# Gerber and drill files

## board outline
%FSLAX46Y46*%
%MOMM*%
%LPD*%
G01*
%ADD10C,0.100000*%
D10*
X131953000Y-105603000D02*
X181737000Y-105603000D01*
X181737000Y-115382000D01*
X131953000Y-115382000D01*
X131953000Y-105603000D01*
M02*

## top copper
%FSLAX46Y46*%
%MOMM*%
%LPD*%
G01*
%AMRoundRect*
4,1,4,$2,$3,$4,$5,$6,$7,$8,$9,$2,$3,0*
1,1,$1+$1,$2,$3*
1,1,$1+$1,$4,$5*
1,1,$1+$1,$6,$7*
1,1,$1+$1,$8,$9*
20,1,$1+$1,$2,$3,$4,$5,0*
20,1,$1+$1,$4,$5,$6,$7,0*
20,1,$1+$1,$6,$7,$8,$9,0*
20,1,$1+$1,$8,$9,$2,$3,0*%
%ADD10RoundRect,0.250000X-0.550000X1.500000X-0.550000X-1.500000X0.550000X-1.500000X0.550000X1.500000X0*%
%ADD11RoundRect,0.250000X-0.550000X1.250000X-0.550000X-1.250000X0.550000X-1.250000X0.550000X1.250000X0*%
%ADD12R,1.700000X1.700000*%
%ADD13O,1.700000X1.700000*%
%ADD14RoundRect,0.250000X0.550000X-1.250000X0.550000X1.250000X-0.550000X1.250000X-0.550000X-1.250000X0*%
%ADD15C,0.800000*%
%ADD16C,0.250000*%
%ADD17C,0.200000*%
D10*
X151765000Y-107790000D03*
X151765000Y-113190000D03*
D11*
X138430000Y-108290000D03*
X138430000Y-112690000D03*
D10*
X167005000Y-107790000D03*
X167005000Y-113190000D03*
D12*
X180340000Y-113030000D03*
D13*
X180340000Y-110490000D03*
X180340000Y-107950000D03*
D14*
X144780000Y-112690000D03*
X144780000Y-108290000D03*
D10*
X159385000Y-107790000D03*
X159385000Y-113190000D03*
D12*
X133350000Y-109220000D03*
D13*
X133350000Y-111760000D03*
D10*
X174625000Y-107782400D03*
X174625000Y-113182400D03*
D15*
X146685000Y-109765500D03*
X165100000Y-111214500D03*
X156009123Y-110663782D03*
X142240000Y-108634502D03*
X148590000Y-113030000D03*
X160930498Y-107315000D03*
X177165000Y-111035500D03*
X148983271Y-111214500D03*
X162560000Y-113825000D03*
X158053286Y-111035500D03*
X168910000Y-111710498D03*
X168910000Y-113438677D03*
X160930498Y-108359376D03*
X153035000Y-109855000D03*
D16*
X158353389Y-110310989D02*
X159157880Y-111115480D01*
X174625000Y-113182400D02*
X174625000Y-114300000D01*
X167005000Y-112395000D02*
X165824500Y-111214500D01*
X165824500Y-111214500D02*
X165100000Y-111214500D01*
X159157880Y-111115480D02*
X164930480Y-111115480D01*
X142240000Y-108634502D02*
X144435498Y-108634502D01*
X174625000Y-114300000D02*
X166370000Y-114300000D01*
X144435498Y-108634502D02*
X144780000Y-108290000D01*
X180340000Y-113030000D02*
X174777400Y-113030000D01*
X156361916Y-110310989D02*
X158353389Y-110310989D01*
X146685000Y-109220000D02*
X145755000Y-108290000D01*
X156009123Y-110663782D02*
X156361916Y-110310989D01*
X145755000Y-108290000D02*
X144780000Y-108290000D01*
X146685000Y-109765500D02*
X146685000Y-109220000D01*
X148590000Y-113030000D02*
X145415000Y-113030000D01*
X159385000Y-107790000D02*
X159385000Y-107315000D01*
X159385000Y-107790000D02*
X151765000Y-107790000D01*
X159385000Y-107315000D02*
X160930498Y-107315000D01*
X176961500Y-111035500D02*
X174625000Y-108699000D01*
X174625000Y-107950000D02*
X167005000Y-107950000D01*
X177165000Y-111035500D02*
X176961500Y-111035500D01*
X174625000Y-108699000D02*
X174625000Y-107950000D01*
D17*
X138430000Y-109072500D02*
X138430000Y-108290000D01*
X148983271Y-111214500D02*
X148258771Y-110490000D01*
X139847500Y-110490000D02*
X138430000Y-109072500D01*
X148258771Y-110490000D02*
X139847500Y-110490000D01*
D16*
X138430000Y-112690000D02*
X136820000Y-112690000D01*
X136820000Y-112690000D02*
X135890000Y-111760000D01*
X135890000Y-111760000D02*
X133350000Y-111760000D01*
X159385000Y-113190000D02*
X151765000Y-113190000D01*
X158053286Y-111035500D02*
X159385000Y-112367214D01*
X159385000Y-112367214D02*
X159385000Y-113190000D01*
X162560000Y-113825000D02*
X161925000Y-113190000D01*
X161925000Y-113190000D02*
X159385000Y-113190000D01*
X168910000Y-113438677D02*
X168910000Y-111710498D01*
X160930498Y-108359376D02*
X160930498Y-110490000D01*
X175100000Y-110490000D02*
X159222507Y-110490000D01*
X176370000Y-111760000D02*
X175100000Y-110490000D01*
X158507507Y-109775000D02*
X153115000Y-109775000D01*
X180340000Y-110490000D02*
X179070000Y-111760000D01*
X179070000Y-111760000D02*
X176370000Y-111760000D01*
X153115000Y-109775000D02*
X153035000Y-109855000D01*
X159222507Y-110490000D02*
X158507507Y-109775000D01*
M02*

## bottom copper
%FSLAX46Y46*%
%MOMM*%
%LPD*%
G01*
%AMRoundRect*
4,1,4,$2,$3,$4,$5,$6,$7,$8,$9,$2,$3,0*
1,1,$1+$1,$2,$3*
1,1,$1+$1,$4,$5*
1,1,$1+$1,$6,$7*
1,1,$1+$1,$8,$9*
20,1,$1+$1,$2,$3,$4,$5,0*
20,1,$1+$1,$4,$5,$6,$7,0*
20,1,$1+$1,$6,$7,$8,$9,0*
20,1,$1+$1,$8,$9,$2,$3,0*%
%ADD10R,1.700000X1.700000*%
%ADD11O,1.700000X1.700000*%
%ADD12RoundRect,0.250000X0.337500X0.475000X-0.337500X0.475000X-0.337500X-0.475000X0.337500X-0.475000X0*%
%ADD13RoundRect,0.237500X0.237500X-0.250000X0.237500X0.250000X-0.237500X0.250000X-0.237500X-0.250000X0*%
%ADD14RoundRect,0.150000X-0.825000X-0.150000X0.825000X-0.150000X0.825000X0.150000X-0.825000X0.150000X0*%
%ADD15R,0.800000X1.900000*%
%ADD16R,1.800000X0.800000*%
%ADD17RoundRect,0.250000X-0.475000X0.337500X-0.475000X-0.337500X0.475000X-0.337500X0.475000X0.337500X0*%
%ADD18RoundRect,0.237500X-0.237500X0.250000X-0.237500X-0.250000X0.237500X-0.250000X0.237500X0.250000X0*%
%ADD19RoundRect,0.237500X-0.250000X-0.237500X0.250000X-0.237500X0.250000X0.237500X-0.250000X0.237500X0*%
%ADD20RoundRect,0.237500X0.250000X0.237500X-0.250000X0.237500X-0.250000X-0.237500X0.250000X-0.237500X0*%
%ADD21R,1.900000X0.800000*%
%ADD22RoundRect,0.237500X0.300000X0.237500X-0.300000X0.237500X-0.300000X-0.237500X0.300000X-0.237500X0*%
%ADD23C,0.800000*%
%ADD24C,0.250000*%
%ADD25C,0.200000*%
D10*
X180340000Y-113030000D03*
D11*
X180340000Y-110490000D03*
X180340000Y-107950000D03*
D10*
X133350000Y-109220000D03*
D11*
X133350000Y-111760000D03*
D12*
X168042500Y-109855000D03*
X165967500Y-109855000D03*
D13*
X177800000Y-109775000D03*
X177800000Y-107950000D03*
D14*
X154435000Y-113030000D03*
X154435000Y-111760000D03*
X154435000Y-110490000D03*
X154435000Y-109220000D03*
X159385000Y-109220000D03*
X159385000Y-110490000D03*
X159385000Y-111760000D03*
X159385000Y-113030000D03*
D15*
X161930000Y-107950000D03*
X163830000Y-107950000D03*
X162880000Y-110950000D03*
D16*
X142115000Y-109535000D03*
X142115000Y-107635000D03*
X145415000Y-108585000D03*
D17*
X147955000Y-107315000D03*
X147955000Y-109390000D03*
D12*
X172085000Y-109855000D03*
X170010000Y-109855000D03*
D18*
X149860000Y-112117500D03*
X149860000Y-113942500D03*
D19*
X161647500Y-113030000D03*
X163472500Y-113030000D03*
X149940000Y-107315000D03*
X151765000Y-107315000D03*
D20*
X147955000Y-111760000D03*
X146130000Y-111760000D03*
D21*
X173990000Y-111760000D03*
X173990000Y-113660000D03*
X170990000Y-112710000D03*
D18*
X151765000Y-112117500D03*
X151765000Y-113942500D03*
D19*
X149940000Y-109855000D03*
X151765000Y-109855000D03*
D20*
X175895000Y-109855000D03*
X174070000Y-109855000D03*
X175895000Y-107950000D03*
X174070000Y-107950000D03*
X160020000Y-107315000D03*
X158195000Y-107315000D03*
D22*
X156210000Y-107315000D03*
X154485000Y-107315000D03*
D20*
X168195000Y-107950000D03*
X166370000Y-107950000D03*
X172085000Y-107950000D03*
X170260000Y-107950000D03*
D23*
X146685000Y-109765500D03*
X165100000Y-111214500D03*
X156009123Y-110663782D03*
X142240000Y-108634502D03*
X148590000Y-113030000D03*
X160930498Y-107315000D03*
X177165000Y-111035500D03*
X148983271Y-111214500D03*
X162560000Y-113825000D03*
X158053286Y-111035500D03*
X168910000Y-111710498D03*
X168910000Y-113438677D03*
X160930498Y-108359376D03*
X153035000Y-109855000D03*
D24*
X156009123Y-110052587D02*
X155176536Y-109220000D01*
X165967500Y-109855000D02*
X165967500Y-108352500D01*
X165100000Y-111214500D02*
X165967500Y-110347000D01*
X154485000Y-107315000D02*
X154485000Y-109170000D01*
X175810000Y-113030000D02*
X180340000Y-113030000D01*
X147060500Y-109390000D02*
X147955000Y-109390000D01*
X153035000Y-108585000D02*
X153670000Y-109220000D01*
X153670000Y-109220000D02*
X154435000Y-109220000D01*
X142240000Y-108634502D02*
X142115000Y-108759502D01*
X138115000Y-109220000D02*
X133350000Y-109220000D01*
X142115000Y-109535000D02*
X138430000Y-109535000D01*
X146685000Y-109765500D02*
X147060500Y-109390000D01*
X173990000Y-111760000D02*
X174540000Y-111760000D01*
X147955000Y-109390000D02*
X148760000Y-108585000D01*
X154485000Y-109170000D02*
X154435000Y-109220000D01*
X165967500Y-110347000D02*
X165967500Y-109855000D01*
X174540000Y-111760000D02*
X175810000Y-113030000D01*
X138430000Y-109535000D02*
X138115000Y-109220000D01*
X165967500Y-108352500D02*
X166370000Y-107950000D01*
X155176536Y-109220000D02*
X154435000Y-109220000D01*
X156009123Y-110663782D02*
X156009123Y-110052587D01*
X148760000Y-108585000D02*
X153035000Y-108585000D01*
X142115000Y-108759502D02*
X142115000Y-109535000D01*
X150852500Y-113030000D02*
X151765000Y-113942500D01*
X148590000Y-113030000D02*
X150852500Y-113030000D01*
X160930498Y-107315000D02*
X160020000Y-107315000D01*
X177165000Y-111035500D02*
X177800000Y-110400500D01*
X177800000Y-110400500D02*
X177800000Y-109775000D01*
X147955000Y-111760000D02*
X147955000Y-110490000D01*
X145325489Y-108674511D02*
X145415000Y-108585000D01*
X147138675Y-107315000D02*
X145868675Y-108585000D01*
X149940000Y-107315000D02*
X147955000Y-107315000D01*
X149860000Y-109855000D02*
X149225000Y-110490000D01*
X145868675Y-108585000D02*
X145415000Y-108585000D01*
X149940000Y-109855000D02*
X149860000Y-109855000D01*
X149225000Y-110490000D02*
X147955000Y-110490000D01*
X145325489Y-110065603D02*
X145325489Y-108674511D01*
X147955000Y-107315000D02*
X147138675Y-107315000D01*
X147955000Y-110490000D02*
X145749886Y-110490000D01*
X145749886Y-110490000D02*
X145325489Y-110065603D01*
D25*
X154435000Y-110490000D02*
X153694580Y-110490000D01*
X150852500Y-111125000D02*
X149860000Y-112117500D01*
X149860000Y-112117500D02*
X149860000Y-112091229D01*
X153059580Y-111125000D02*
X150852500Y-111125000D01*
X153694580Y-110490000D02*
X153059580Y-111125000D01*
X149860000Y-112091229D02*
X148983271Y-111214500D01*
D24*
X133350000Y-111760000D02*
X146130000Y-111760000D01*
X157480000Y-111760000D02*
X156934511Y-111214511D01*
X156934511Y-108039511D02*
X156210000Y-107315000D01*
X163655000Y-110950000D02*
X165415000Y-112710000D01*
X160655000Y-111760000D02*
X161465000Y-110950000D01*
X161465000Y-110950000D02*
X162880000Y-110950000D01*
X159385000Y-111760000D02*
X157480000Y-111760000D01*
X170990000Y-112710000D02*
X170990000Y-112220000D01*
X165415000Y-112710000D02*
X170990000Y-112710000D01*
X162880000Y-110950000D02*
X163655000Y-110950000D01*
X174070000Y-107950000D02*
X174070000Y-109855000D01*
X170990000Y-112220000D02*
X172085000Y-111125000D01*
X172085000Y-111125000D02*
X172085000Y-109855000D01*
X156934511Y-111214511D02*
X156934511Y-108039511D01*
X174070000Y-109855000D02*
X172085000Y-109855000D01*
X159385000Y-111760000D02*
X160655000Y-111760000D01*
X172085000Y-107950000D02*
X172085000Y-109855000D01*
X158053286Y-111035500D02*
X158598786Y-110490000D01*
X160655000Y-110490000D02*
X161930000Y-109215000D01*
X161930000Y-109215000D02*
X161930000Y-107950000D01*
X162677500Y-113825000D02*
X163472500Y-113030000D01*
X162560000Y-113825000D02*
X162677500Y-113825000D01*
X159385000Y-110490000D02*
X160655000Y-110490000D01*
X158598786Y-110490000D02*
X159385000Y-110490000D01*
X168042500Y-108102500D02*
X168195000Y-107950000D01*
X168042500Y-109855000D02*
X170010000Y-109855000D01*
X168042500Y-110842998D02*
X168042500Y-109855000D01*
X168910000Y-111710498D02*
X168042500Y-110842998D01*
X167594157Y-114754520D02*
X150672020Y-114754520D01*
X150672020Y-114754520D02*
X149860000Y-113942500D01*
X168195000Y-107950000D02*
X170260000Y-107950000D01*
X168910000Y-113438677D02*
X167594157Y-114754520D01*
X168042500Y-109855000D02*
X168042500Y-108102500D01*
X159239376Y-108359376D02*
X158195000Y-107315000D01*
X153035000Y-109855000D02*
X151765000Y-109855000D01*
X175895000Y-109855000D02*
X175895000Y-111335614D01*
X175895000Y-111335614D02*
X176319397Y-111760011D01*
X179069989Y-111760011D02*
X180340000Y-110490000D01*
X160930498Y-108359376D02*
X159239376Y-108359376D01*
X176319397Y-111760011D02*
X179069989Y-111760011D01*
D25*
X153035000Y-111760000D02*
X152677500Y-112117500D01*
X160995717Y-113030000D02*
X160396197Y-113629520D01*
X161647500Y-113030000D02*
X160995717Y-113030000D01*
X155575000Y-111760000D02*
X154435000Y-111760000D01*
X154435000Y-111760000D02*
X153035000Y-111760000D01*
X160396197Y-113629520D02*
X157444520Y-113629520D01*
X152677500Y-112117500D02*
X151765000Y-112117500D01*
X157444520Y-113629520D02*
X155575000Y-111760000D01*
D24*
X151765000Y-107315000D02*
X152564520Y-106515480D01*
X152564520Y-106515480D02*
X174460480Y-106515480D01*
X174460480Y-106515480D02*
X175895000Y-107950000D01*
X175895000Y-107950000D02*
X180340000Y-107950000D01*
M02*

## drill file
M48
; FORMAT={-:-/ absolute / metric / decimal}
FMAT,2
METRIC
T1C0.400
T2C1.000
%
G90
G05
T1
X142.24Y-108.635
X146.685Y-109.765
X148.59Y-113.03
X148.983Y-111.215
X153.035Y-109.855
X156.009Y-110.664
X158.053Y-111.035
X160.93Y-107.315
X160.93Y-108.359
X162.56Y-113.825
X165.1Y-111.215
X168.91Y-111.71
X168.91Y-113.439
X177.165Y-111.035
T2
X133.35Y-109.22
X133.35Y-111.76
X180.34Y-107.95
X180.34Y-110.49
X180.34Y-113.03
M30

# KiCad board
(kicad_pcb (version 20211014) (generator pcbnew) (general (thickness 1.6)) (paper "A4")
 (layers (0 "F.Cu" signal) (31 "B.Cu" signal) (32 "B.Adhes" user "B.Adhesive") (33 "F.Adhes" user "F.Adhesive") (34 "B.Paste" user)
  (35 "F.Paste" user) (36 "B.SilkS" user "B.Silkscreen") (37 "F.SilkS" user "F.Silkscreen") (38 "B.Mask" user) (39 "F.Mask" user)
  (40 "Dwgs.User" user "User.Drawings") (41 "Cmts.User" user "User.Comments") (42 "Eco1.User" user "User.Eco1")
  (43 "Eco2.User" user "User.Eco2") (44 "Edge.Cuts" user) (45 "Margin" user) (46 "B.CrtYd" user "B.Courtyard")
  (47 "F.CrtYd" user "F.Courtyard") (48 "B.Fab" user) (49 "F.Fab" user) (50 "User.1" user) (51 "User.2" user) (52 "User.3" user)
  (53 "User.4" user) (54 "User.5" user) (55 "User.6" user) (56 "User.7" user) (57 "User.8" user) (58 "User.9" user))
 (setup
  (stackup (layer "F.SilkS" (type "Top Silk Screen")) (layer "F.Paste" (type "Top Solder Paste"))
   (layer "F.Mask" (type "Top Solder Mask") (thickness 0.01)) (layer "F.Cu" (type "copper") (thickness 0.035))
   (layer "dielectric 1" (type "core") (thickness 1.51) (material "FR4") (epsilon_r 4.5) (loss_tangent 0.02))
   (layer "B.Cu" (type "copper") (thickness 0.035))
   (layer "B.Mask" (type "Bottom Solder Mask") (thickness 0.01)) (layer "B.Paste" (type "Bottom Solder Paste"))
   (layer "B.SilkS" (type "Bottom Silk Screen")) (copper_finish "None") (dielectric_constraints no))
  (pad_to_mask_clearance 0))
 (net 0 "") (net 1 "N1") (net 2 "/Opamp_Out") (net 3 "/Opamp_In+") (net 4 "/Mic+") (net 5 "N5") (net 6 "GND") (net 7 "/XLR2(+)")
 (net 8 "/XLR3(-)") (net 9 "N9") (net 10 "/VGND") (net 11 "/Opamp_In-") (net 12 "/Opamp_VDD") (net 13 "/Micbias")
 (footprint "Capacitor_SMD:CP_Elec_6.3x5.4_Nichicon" (layer "F.Cu") (at 151.765 110.49 -90)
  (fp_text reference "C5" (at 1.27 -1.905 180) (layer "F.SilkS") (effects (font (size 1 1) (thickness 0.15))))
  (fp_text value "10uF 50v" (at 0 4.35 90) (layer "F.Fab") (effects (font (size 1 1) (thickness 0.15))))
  (pad "1" smd roundrect (at -2.7 0 270) (size 3.5 1.6) (layers "F.Cu" "F.Paste" "F.Mask") (roundrect_rratio 0.15625) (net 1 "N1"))
  (pad "2" smd roundrect (at 2.7 0 270) (size 3.5 1.6) (layers "F.Cu" "F.Paste" "F.Mask") (roundrect_rratio 0.15625) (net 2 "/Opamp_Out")))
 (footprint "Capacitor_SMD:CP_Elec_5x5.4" (layer "F.Cu") (at 138.43 110.49 -90)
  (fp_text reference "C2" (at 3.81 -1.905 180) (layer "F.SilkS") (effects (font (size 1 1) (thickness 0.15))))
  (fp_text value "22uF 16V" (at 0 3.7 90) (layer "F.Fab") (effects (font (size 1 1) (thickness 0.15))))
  (pad "1" smd roundrect (at -2.2 0 270) (size 3 1.6) (layers "F.Cu" "F.Paste" "F.Mask") (roundrect_rratio 0.15625) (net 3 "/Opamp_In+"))
  (pad "2" smd roundrect (at 2.2 0 270) (size 3 1.6) (layers "F.Cu" "F.Paste" "F.Mask") (roundrect_rratio 0.15625) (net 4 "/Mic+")))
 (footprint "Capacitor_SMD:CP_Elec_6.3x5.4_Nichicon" (layer "F.Cu") (at 167.005 110.49 -90)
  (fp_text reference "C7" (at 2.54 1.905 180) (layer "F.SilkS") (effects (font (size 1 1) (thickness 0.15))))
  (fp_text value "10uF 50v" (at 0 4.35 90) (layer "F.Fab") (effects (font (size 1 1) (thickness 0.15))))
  (pad "1" smd roundrect (at -2.7 0 270) (size 3.5 1.6) (layers "F.Cu" "F.Paste" "F.Mask") (roundrect_rratio 0.15625) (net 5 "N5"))
  (pad "2" smd roundrect (at 2.7 0 270) (size 3.5 1.6) (layers "F.Cu" "F.Paste" "F.Mask") (roundrect_rratio 0.15625) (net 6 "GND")))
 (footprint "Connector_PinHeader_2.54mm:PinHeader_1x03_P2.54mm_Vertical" (layer "F.Cu") (at 180.34 113.03 180)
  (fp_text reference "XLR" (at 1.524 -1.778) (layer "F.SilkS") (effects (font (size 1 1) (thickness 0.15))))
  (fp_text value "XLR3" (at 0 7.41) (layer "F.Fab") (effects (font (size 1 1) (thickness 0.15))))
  (pad "1" thru_hole rect (at 0 0 180) (size 1.7 1.7) (drill 1) (layers *.Cu *.Mask) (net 6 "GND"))
  (pad "2" thru_hole oval (at 0 2.54 180) (size 1.7 1.7) (drill 1) (layers *.Cu *.Mask) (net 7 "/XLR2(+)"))
  (pad "3" thru_hole oval (at 0 5.08 180) (size 1.7 1.7) (drill 1) (layers *.Cu *.Mask) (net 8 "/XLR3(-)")))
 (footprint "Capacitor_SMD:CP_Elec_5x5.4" (layer "F.Cu") (at 144.78 110.49 90)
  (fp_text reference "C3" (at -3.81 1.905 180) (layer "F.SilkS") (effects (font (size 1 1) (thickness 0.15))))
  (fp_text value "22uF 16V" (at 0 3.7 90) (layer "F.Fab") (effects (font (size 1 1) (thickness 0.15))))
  (pad "1" smd roundrect (at -2.2 0 90) (size 3 1.6) (layers "F.Cu" "F.Paste" "F.Mask") (roundrect_rratio 0.15625) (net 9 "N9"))
  (pad "2" smd roundrect (at 2.2 0 90) (size 3 1.6) (layers "F.Cu" "F.Paste" "F.Mask") (roundrect_rratio 0.15625) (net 6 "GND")))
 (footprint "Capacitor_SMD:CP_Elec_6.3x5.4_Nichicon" (layer "F.Cu") (at 159.385 110.49 -90)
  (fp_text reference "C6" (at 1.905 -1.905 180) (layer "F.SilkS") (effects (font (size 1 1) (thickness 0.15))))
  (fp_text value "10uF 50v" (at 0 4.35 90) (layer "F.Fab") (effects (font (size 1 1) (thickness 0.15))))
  (pad "1" smd roundrect (at -2.7 0 270) (size 3.5 1.6) (layers "F.Cu" "F.Paste" "F.Mask") (roundrect_rratio 0.15625) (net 1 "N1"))
  (pad "2" smd roundrect (at 2.7 0 270) (size 3.5 1.6) (layers "F.Cu" "F.Paste" "F.Mask") (roundrect_rratio 0.15625) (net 2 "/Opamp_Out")))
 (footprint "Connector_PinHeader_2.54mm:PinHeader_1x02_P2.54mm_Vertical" (layer "F.Cu") (at 133.35 109.22)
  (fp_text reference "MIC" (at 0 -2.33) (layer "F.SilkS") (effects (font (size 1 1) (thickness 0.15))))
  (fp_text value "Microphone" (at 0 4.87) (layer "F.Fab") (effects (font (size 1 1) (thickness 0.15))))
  (pad "1" thru_hole rect (at 0 0) (size 1.7 1.7) (drill 1) (layers *.Cu *.Mask) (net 6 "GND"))
  (pad "2" thru_hole oval (at 0 2.54) (size 1.7 1.7) (drill 1) (layers *.Cu *.Mask) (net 4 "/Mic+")))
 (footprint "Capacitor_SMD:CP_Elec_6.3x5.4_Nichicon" (layer "F.Cu") (at 174.625 110.4824 -90)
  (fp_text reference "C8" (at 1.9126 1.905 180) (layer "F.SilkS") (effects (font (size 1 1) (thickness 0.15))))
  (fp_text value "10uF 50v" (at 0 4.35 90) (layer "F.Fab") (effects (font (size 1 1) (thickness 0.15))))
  (pad "1" smd roundrect (at -2.7 0 270) (size 3.5 1.6) (layers "F.Cu" "F.Paste" "F.Mask") (roundrect_rratio 0.15625) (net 5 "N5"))
  (pad "2" smd roundrect (at 2.7 0 270) (size 3.5 1.6) (layers "F.Cu" "F.Paste" "F.Mask") (roundrect_rratio 0.15625) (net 6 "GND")))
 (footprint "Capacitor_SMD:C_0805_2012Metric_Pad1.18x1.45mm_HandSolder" (layer "B.Cu") (at 167.005 109.855 180)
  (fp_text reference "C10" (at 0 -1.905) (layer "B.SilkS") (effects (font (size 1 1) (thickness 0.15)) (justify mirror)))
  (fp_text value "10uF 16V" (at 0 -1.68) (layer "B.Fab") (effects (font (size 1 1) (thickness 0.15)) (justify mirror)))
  (pad "1" smd roundrect (at -1.0375 0 180) (size 1.175 1.45) (layers "B.Cu" "B.Paste" "B.Mask") (roundrect_rratio 0.2127659574)
   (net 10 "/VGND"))
  (pad "2" smd roundrect (at 1.0375 0 180) (size 1.175 1.45) (layers "B.Cu" "B.Paste" "B.Mask") (roundrect_rratio 0.2127659574)
   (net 6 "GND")))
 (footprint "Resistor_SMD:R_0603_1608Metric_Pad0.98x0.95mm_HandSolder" (layer "B.Cu") (at 177.8 108.8625 90)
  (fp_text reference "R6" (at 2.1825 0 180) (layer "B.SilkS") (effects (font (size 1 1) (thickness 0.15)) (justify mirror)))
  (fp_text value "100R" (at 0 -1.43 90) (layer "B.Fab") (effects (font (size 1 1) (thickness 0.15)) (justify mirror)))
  (pad "1" smd roundrect (at -0.9125 0 90) (size 0.975 0.95) (layers "B.Cu" "B.Paste" "B.Mask") (roundrect_rratio 0.25) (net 5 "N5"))
  (pad "2" smd roundrect (at 0.9125 0 90) (size 0.975 0.95) (layers "B.Cu" "B.Paste" "B.Mask") (roundrect_rratio 0.25) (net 8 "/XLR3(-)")))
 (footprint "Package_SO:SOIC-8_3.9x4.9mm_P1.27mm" (layer "B.Cu") (at 156.91 111.125)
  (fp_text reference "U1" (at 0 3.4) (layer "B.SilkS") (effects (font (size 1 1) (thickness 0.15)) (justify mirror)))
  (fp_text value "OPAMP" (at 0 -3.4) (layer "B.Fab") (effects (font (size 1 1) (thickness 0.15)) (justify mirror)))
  (pad "1" smd roundrect (at -2.475 1.905) (size 1.95 0.6) (layers "B.Cu" "B.Paste" "B.Mask") (roundrect_rratio 0.25))
  (pad "2" smd roundrect (at -2.475 0.635) (size 1.95 0.6) (layers "B.Cu" "B.Paste" "B.Mask") (roundrect_rratio 0.25) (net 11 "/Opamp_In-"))
  (pad "3" smd roundrect (at -2.475 -0.635) (size 1.95 0.6) (layers "B.Cu" "B.Paste" "B.Mask") (roundrect_rratio 0.25) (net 3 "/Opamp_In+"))
  (pad "4" smd roundrect (at -2.475 -1.905) (size 1.95 0.6) (layers "B.Cu" "B.Paste" "B.Mask") (roundrect_rratio 0.25) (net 6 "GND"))
  (pad "5" smd roundrect (at 2.475 -1.905) (size 1.95 0.6) (layers "B.Cu" "B.Paste" "B.Mask") (roundrect_rratio 0.25))
  (pad "6" smd roundrect (at 2.475 -0.635) (size 1.95 0.6) (layers "B.Cu" "B.Paste" "B.Mask") (roundrect_rratio 0.25) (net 2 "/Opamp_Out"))
  (pad "7" smd roundrect (at 2.475 0.635) (size 1.95 0.6) (layers "B.Cu" "B.Paste" "B.Mask") (roundrect_rratio 0.25) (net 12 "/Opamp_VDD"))
  (pad "8" smd roundrect (at 2.475 1.905) (size 1.95 0.6) (layers "B.Cu" "B.Paste" "B.Mask") (roundrect_rratio 0.25)))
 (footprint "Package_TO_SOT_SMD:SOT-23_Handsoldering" (layer "B.Cu") (at 162.88 109.45 -90)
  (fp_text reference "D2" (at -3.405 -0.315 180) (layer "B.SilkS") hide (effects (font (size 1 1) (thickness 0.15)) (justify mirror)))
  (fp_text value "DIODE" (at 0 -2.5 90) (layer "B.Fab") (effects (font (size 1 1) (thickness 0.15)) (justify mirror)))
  (pad "1" smd rect (at -1.5 0.95 270) (size 1.9 0.8) (layers "B.Cu" "B.Paste" "B.Mask") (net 2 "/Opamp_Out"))
  (pad "2" smd rect (at -1.5 -0.95 270) (size 1.9 0.8) (layers "B.Cu" "B.Paste" "B.Mask"))
  (pad "3" smd rect (at 1.5 0 270) (size 1.9 0.8) (layers "B.Cu" "B.Paste" "B.Mask") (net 12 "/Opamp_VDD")))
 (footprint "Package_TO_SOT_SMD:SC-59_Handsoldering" (layer "B.Cu") (at 143.765 108.585)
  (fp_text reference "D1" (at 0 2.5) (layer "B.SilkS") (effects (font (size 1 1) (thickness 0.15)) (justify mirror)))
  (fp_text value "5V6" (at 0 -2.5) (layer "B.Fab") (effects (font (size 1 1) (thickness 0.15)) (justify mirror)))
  (pad "1" smd rect (at -1.65 0.95) (size 1.8 0.8) (layers "B.Cu" "B.Paste" "B.Mask") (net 6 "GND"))
  (pad "2" smd rect (at -1.65 -0.95) (size 1.8 0.8) (layers "B.Cu" "B.Paste" "B.Mask"))
  (pad "3" smd rect (at 1.65 0) (size 1.8 0.8) (layers "B.Cu" "B.Paste" "B.Mask") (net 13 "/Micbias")))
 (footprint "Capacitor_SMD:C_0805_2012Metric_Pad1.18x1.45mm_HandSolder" (layer "B.Cu") (at 147.955 108.3525 -90)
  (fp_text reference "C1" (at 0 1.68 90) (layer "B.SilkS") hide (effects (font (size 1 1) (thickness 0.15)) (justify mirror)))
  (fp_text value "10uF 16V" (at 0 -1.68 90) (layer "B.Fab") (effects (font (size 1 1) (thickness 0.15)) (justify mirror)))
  (pad "1" smd roundrect (at -1.0375 0 270) (size 1.175 1.45) (layers "B.Cu" "B.Paste" "B.Mask") (roundrect_rratio 0.2127659574)
   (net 13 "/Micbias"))
  (pad "2" smd roundrect (at 1.0375 0 270) (size 1.175 1.45) (layers "B.Cu" "B.Paste" "B.Mask") (roundrect_rratio 0.2127659574)
   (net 6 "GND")))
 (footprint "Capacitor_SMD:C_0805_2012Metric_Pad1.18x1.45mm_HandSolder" (layer "B.Cu") (at 171.0475 109.855 180)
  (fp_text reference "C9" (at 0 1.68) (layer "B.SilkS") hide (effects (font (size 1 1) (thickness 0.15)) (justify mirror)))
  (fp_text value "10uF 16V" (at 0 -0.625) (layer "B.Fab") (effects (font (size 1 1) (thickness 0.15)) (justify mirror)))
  (pad "1" smd roundrect (at -1.0375 0 180) (size 1.175 1.45) (layers "B.Cu" "B.Paste" "B.Mask") (roundrect_rratio 0.2127659574)
   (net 12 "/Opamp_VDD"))
  (pad "2" smd roundrect (at 1.0375 0 180) (size 1.175 1.45) (layers "B.Cu" "B.Paste" "B.Mask") (roundrect_rratio 0.2127659574)
   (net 10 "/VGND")))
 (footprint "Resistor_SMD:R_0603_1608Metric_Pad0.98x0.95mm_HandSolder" (layer "B.Cu") (at 149.86 113.03 -90)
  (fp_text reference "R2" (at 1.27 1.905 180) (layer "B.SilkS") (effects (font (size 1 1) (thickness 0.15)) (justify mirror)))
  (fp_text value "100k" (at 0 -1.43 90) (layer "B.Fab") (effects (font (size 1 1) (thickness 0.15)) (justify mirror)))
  (pad "1" smd roundrect (at -0.9125 0 270) (size 0.975 0.95) (layers "B.Cu" "B.Paste" "B.Mask") (roundrect_rratio 0.25)
   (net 3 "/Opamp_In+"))
  (pad "2" smd roundrect (at 0.9125 0 270) (size 0.975 0.95) (layers "B.Cu" "B.Paste" "B.Mask") (roundrect_rratio 0.25) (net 10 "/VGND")))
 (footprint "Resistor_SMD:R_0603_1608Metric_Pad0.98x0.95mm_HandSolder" (layer "B.Cu") (at 162.56 113.03)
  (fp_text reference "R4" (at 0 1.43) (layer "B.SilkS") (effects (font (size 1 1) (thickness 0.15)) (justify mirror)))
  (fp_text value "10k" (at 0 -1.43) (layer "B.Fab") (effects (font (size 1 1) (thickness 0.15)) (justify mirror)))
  (pad "1" smd roundrect (at -0.9125 0) (size 0.975 0.95) (layers "B.Cu" "B.Paste" "B.Mask") (roundrect_rratio 0.25) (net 11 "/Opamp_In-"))
  (pad "2" smd roundrect (at 0.9125 0) (size 0.975 0.95) (layers "B.Cu" "B.Paste" "B.Mask") (roundrect_rratio 0.25) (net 2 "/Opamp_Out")))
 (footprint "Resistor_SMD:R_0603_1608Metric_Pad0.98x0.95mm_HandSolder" (layer "B.Cu") (at 150.8525 107.315)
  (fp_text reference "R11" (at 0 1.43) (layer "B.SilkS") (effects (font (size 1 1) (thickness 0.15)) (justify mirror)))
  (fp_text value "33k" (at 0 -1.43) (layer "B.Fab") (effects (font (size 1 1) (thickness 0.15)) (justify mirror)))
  (pad "1" smd roundrect (at -0.9125 0) (size 0.975 0.95) (layers "B.Cu" "B.Paste" "B.Mask") (roundrect_rratio 0.25) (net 13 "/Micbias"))
  (pad "2" smd roundrect (at 0.9125 0) (size 0.975 0.95) (layers "B.Cu" "B.Paste" "B.Mask") (roundrect_rratio 0.25) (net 8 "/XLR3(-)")))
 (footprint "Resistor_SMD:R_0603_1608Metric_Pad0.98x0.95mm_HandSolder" (layer "B.Cu") (at 147.0425 111.76 180)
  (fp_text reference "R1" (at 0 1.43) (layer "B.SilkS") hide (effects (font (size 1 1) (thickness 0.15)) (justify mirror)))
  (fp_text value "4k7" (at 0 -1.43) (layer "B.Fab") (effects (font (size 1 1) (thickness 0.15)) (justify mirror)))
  (pad "1" smd roundrect (at -0.9125 0 180) (size 0.975 0.95) (layers "B.Cu" "B.Paste" "B.Mask") (roundrect_rratio 0.25) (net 13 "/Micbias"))
  (pad "2" smd roundrect (at 0.9125 0 180) (size 0.975 0.95) (layers "B.Cu" "B.Paste" "B.Mask") (roundrect_rratio 0.25) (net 4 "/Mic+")))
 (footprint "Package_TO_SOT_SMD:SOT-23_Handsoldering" (layer "B.Cu") (at 172.49 112.71 180)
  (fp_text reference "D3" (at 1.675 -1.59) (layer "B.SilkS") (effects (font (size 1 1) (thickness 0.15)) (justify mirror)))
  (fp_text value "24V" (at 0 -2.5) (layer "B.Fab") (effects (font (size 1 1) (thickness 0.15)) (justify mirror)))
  (pad "1" smd rect (at -1.5 0.95 180) (size 1.9 0.8) (layers "B.Cu" "B.Paste" "B.Mask") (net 6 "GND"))
  (pad "2" smd rect (at -1.5 -0.95 180) (size 1.9 0.8) (layers "B.Cu" "B.Paste" "B.Mask"))
  (pad "3" smd rect (at 1.5 0 180) (size 1.9 0.8) (layers "B.Cu" "B.Paste" "B.Mask") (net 12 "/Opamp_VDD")))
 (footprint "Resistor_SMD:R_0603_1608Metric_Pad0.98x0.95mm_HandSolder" (layer "B.Cu") (at 151.765 113.03 -90)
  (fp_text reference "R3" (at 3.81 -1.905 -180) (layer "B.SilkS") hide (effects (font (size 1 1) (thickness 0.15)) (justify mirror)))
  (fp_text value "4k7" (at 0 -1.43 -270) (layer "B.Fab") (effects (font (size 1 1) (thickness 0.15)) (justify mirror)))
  (pad "1" smd roundrect (at -0.9125 0 270) (size 0.975 0.95) (layers "B.Cu" "B.Paste" "B.Mask") (roundrect_rratio 0.25)
   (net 11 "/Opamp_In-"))
  (pad "2" smd roundrect (at 0.9125 0 270) (size 0.975 0.95) (layers "B.Cu" "B.Paste" "B.Mask") (roundrect_rratio 0.25) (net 9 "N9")))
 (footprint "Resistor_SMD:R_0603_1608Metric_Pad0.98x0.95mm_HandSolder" (layer "B.Cu") (at 150.8525 109.855)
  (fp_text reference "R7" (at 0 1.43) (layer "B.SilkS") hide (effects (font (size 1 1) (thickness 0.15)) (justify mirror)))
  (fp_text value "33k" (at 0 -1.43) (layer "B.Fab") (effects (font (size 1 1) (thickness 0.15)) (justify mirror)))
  (pad "1" smd roundrect (at -0.9125 0) (size 0.975 0.95) (layers "B.Cu" "B.Paste" "B.Mask") (roundrect_rratio 0.25) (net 13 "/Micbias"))
  (pad "2" smd roundrect (at 0.9125 0) (size 0.975 0.95) (layers "B.Cu" "B.Paste" "B.Mask") (roundrect_rratio 0.25) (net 7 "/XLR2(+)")))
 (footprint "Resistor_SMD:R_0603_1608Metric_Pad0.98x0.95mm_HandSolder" (layer "B.Cu") (at 174.9825 109.855 180)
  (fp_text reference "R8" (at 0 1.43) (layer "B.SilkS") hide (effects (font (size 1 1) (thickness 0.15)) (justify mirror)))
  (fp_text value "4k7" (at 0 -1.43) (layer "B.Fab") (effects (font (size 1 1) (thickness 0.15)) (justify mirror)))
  (pad "1" smd roundrect (at -0.9125 0 180) (size 0.975 0.95) (layers "B.Cu" "B.Paste" "B.Mask") (roundrect_rratio 0.25) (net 7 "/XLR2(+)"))
  (pad "2" smd roundrect (at 0.9125 0 180) (size 0.975 0.95) (layers "B.Cu" "B.Paste" "B.Mask") (roundrect_rratio 0.25)
   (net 12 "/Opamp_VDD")))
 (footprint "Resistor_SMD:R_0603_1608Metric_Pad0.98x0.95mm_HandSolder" (layer "B.Cu") (at 174.9825 107.95 180)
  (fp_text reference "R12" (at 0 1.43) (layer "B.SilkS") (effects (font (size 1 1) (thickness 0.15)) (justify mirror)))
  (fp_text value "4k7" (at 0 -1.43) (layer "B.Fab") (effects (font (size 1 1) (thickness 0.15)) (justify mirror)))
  (pad "1" smd roundrect (at -0.9125 0 180) (size 0.975 0.95) (layers "B.Cu" "B.Paste" "B.Mask") (roundrect_rratio 0.25) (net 8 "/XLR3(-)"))
  (pad "2" smd roundrect (at 0.9125 0 180) (size 0.975 0.95) (layers "B.Cu" "B.Paste" "B.Mask") (roundrect_rratio 0.25)
   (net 12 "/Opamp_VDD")))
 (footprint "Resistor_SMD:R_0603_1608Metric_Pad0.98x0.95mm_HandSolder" (layer "B.Cu") (at 159.1075 107.315 180)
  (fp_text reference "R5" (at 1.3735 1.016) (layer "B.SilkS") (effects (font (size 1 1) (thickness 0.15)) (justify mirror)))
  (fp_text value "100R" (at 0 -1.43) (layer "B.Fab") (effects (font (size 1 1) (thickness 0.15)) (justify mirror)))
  (pad "1" smd roundrect (at -0.9125 0 180) (size 0.975 0.95) (layers "B.Cu" "B.Paste" "B.Mask") (roundrect_rratio 0.25) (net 1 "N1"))
  (pad "2" smd roundrect (at 0.9125 0 180) (size 0.975 0.95) (layers "B.Cu" "B.Paste" "B.Mask") (roundrect_rratio 0.25) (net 7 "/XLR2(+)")))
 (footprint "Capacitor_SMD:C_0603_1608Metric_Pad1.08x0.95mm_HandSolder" (layer "B.Cu") (at 155.3475 107.315 180)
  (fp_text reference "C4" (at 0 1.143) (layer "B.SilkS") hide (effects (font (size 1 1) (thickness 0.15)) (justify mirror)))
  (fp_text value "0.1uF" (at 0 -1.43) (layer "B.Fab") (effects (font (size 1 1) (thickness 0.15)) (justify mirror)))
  (pad "1" smd roundrect (at -0.8625 0 180) (size 1.075 0.95) (layers "B.Cu" "B.Paste" "B.Mask") (roundrect_rratio 0.25)
   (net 12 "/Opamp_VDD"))
  (pad "2" smd roundrect (at 0.8625 0 180) (size 1.075 0.95) (layers "B.Cu" "B.Paste" "B.Mask") (roundrect_rratio 0.25) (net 6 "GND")))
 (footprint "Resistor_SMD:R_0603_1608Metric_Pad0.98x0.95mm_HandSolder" (layer "B.Cu") (at 167.2825 107.95 180)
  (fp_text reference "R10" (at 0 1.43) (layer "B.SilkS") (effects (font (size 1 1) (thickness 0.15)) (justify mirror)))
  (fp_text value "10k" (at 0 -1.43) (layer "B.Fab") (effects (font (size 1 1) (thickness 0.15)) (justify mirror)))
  (pad "1" smd roundrect (at -0.9125 0 180) (size 0.975 0.95) (layers "B.Cu" "B.Paste" "B.Mask") (roundrect_rratio 0.25) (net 10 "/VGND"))
  (pad "2" smd roundrect (at 0.9125 0 180) (size 0.975 0.95) (layers "B.Cu" "B.Paste" "B.Mask") (roundrect_rratio 0.25) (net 6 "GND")))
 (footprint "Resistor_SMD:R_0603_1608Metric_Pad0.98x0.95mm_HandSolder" (layer "B.Cu") (at 171.1725 107.95 180)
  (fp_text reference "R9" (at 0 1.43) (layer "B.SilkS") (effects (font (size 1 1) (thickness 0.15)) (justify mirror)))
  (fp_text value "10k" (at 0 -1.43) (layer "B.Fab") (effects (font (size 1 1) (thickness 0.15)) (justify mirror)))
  (pad "1" smd roundrect (at -0.9125 0 180) (size 0.975 0.95) (layers "B.Cu" "B.Paste" "B.Mask") (roundrect_rratio 0.25)
   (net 12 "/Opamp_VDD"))
  (pad "2" smd roundrect (at 0.9125 0 180) (size 0.975 0.95) (layers "B.Cu" "B.Paste" "B.Mask") (roundrect_rratio 0.25) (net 10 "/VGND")))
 (gr_rect (start 131.953 105.603) (end 181.737 115.382) (layer "Edge.Cuts") (width 0.1) (fill none))
 (segment (start 158.353389 110.310989) (end 159.15788 111.11548) (width 0.25) (layer "F.Cu") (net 6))
 (segment (start 174.625 113.1824) (end 174.625 114.3) (width 0.25) (layer "F.Cu") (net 6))
 (segment (start 167.005 112.395) (end 165.8245 111.2145) (width 0.25) (layer "F.Cu") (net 6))
 (segment (start 165.8245 111.2145) (end 165.1 111.2145) (width 0.25) (layer "F.Cu") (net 6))
 (segment (start 159.15788 111.11548) (end 164.93048 111.11548) (width 0.25) (layer "F.Cu") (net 6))
 (segment (start 142.24 108.634502) (end 144.435498 108.634502) (width 0.25) (layer "F.Cu") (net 6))
 (segment (start 174.625 114.3) (end 166.37 114.3) (width 0.25) (layer "F.Cu") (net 6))
 (segment (start 144.435498 108.634502) (end 144.78 108.29) (width 0.25) (layer "F.Cu") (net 6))
 (segment (start 180.34 113.03) (end 174.7774 113.03) (width 0.25) (layer "F.Cu") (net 6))
 (segment (start 156.361916 110.310989) (end 158.353389 110.310989) (width 0.25) (layer "F.Cu") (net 6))
 (segment (start 146.685 109.22) (end 145.755 108.29) (width 0.25) (layer "F.Cu") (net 6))
 (segment (start 156.009123 110.663782) (end 156.361916 110.310989) (width 0.25) (layer "F.Cu") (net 6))
 (segment (start 145.755 108.29) (end 144.78 108.29) (width 0.25) (layer "F.Cu") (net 6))
 (segment (start 146.685 109.7655) (end 146.685 109.22) (width 0.25) (layer "F.Cu") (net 6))
 (via (at 146.685 109.7655) (size 0.8) (drill 0.4) (layers "F.Cu" "B.Cu") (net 6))
 (via (at 165.1 111.2145) (size 0.8) (drill 0.4) (layers "F.Cu" "B.Cu") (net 6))
 (via (at 156.009123 110.663782) (size 0.8) (drill 0.4) (layers "F.Cu" "B.Cu") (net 6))
 (via (at 142.24 108.634502) (size 0.8) (drill 0.4) (layers "F.Cu" "B.Cu") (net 6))
 (segment (start 156.009123 110.052587) (end 155.176536 109.22) (width 0.25) (layer "B.Cu") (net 6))
 (segment (start 165.9675 109.855) (end 165.9675 108.3525) (width 0.25) (layer "B.Cu") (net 6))
 (segment (start 165.1 111.2145) (end 165.9675 110.347) (width 0.25) (layer "B.Cu") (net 6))
 (segment (start 154.485 107.315) (end 154.485 109.17) (width 0.25) (layer "B.Cu") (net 6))
 (segment (start 175.81 113.03) (end 180.34 113.03) (width 0.25) (layer "B.Cu") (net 6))
 (segment (start 147.0605 109.39) (end 147.955 109.39) (width 0.25) (layer "B.Cu") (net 6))
 (segment (start 153.035 108.585) (end 153.67 109.22) (width 0.25) (layer "B.Cu") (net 6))
 (segment (start 153.67 109.22) (end 154.435 109.22) (width 0.25) (layer "B.Cu") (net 6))
 (segment (start 142.24 108.634502) (end 142.115 108.759502) (width 0.25) (layer "B.Cu") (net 6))
 (segment (start 138.115 109.22) (end 133.35 109.22) (width 0.25) (layer "B.Cu") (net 6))
 (segment (start 142.115 109.535) (end 138.43 109.535) (width 0.25) (layer "B.Cu") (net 6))
 (segment (start 146.685 109.7655) (end 147.0605 109.39) (width 0.25) (layer "B.Cu") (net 6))
 (segment (start 173.99 111.76) (end 174.54 111.76) (width 0.25) (layer "B.Cu") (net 6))
 (segment (start 147.955 109.39) (end 148.76 108.585) (width 0.25) (layer "B.Cu") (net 6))
 (segment (start 154.485 109.17) (end 154.435 109.22) (width 0.25) (layer "B.Cu") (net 6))
 (segment (start 165.9675 110.347) (end 165.9675 109.855) (width 0.25) (layer "B.Cu") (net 6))
 (segment (start 174.54 111.76) (end 175.81 113.03) (width 0.25) (layer "B.Cu") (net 6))
 (segment (start 138.43 109.535) (end 138.115 109.22) (width 0.25) (layer "B.Cu") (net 6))
 (segment (start 165.9675 108.3525) (end 166.37 107.95) (width 0.25) (layer "B.Cu") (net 6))
 (segment (start 155.176536 109.22) (end 154.435 109.22) (width 0.25) (layer "B.Cu") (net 6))
 (segment (start 156.009123 110.663782) (end 156.009123 110.052587) (width 0.25) (layer "B.Cu") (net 6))
 (segment (start 148.76 108.585) (end 153.035 108.585) (width 0.25) (layer "B.Cu") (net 6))
 (segment (start 142.115 108.759502) (end 142.115 109.535) (width 0.25) (layer "B.Cu") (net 6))
 (segment (start 148.59 113.03) (end 145.415 113.03) (width 0.25) (layer "F.Cu") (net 9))
 (via (at 148.59 113.03) (size 0.8) (drill 0.4) (layers "F.Cu" "B.Cu") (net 9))
 (segment (start 150.8525 113.03) (end 151.765 113.9425) (width 0.25) (layer "B.Cu") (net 9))
 (segment (start 148.59 113.03) (end 150.8525 113.03) (width 0.25) (layer "B.Cu") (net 9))
 (segment (start 159.385 107.79) (end 159.385 107.315) (width 0.25) (layer "F.Cu") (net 1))
 (segment (start 159.385 107.79) (end 151.765 107.79) (width 0.25) (layer "F.Cu") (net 1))
 (segment (start 159.385 107.315) (end 160.930498 107.315) (width 0.25) (layer "F.Cu") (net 1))
 (via (at 160.930498 107.315) (size 0.8) (drill 0.4) (layers "F.Cu" "B.Cu") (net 1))
 (segment (start 160.930498 107.315) (end 160.02 107.315) (width 0.25) (layer "B.Cu") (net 1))
 (segment (start 176.9615 111.0355) (end 174.625 108.699) (width 0.25) (layer "F.Cu") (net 5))
 (segment (start 174.625 107.95) (end 167.005 107.95) (width 0.25) (layer "F.Cu") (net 5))
 (segment (start 177.165 111.0355) (end 176.9615 111.0355) (width 0.25) (layer "F.Cu") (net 5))
 (segment (start 174.625 108.699) (end 174.625 107.95) (width 0.25) (layer "F.Cu") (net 5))
 (via (at 177.165 111.0355) (size 0.8) (drill 0.4) (layers "F.Cu" "B.Cu") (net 5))
 (segment (start 177.165 111.0355) (end 177.8 110.4005) (width 0.25) (layer "B.Cu") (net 5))
 (segment (start 177.8 110.4005) (end 177.8 109.775) (width 0.25) (layer "B.Cu") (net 5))
 (segment (start 147.955 111.76) (end 147.955 110.49) (width 0.25) (layer "B.Cu") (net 13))
 (segment (start 145.325489 108.674511) (end 145.415 108.585) (width 0.25) (layer "B.Cu") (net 13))
 (segment (start 147.138675 107.315) (end 145.868675 108.585) (width 0.25) (layer "B.Cu") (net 13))
 (segment (start 149.94 107.315) (end 147.955 107.315) (width 0.25) (layer "B.Cu") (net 13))
 (segment (start 149.86 109.855) (end 149.225 110.49) (width 0.25) (layer "B.Cu") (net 13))
 (segment (start 145.868675 108.585) (end 145.415 108.585) (width 0.25) (layer "B.Cu") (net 13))
 (segment (start 149.94 109.855) (end 149.86 109.855) (width 0.25) (layer "B.Cu") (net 13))
 (segment (start 149.225 110.49) (end 147.955 110.49) (width 0.25) (layer "B.Cu") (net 13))
 (segment (start 145.325489 110.065603) (end 145.325489 108.674511) (width 0.25) (layer "B.Cu") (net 13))
 (segment (start 147.955 107.315) (end 147.138675 107.315) (width 0.25) (layer "B.Cu") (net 13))
 (segment (start 147.955 110.49) (end 145.749886 110.49) (width 0.25) (layer "B.Cu") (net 13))
 (segment (start 145.749886 110.49) (end 145.325489 110.065603) (width 0.25) (layer "B.Cu") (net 13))
 (segment (start 138.43 109.0725) (end 138.43 108.29) (width 0.2) (layer "F.Cu") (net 3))
 (segment (start 148.983271 111.2145) (end 148.258771 110.49) (width 0.2) (layer "F.Cu") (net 3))
 (segment (start 139.8475 110.49) (end 138.43 109.0725) (width 0.2) (layer "F.Cu") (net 3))
 (segment (start 148.258771 110.49) (end 139.8475 110.49) (width 0.2) (layer "F.Cu") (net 3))
 (via (at 148.983271 111.2145) (size 0.8) (drill 0.4) (layers "F.Cu" "B.Cu") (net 3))
 (segment (start 154.435 110.49) (end 153.69458 110.49) (width 0.2) (layer "B.Cu") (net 3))
 (segment (start 150.8525 111.125) (end 149.86 112.1175) (width 0.2) (layer "B.Cu") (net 3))
 (segment (start 149.86 112.1175) (end 149.86 112.091229) (width 0.2) (layer "B.Cu") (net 3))
 (segment (start 153.05958 111.125) (end 150.8525 111.125) (width 0.2) (layer "B.Cu") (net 3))
 (segment (start 153.69458 110.49) (end 153.05958 111.125) (width 0.2) (layer "B.Cu") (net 3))
 (segment (start 149.86 112.091229) (end 148.983271 111.2145) (width 0.2) (layer "B.Cu") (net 3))
 (segment (start 138.43 112.69) (end 136.82 112.69) (width 0.25) (layer "F.Cu") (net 4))
 (segment (start 136.82 112.69) (end 135.89 111.76) (width 0.25) (layer "F.Cu") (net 4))
 (segment (start 135.89 111.76) (end 133.35 111.76) (width 0.25) (layer "F.Cu") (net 4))
 (segment (start 133.35 111.76) (end 146.13 111.76) (width 0.25) (layer "B.Cu") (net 4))
 (segment (start 157.48 111.76) (end 156.934511 111.214511) (width 0.25) (layer "B.Cu") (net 12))
 (segment (start 156.934511 108.039511) (end 156.21 107.315) (width 0.25) (layer "B.Cu") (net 12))
 (segment (start 163.655 110.95) (end 165.415 112.71) (width 0.25) (layer "B.Cu") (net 12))
 (segment (start 160.655 111.76) (end 161.465 110.95) (width 0.25) (layer "B.Cu") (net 12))
 (segment (start 161.465 110.95) (end 162.88 110.95) (width 0.25) (layer "B.Cu") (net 12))
 (segment (start 159.385 111.76) (end 157.48 111.76) (width 0.25) (layer "B.Cu") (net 12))
 (segment (start 170.99 112.71) (end 170.99 112.22) (width 0.25) (layer "B.Cu") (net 12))
 (segment (start 165.415 112.71) (end 170.99 112.71) (width 0.25) (layer "B.Cu") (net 12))
 (segment (start 162.88 110.95) (end 163.655 110.95) (width 0.25) (layer "B.Cu") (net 12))
 (segment (start 174.07 107.95) (end 174.07 109.855) (width 0.25) (layer "B.Cu") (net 12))
 (segment (start 170.99 112.22) (end 172.085 111.125) (width 0.25) (layer "B.Cu") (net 12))
 (segment (start 172.085 111.125) (end 172.085 109.855) (width 0.25) (layer "B.Cu") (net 12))
 (segment (start 156.934511 111.214511) (end 156.934511 108.039511) (width 0.25) (layer "B.Cu") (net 12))
 (segment (start 174.07 109.855) (end 172.085 109.855) (width 0.25) (layer "B.Cu") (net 12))
 (segment (start 159.385 111.76) (end 160.655 111.76) (width 0.25) (layer "B.Cu") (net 12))
 (segment (start 172.085 107.95) (end 172.085 109.855) (width 0.25) (layer "B.Cu") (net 12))
 (segment (start 159.385 113.19) (end 151.765 113.19) (width 0.25) (layer "F.Cu") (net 2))
 (segment (start 158.053286 111.0355) (end 159.385 112.367214) (width 0.25) (layer "F.Cu") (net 2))
 (segment (start 159.385 112.367214) (end 159.385 113.19) (width 0.25) (layer "F.Cu") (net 2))
 (segment (start 162.56 113.825) (end 161.925 113.19) (width 0.25) (layer "F.Cu") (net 2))
 (segment (start 161.925 113.19) (end 159.385 113.19) (width 0.25) (layer "F.Cu") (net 2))
 (via (at 162.56 113.825) (size 0.8) (drill 0.4) (layers "F.Cu" "B.Cu") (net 2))
 (via (at 158.053286 111.0355) (size 0.8) (drill 0.4) (layers "F.Cu" "B.Cu") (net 2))
 (segment (start 158.053286 111.0355) (end 158.598786 110.49) (width 0.25) (layer "B.Cu") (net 2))
 (segment (start 160.655 110.49) (end 161.93 109.215) (width 0.25) (layer "B.Cu") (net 2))
 (segment (start 161.93 109.215) (end 161.93 107.95) (width 0.25) (layer "B.Cu") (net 2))
 (segment (start 162.6775 113.825) (end 163.4725 113.03) (width 0.25) (layer "B.Cu") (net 2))
 (segment (start 162.56 113.825) (end 162.6775 113.825) (width 0.25) (layer "B.Cu") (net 2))
 (segment (start 159.385 110.49) (end 160.655 110.49) (width 0.25) (layer "B.Cu") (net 2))
 (segment (start 158.598786 110.49) (end 159.385 110.49) (width 0.25) (layer "B.Cu") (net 2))
 (segment (start 168.91 113.438677) (end 168.91 111.710498) (width 0.25) (layer "F.Cu") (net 10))
 (via (at 168.91 111.710498) (size 0.8) (drill 0.4) (layers "F.Cu" "B.Cu") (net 10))
 (via (at 168.91 113.438677) (size 0.8) (drill 0.4) (layers "F.Cu" "B.Cu") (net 10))
 (segment (start 168.0425 108.1025) (end 168.195 107.95) (width 0.25) (layer "B.Cu") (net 10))
 (segment (start 168.0425 109.855) (end 170.01 109.855) (width 0.25) (layer "B.Cu") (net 10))
 (segment (start 168.0425 110.842998) (end 168.0425 109.855) (width 0.25) (layer "B.Cu") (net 10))
 (segment (start 168.91 111.710498) (end 168.0425 110.842998) (width 0.25) (layer "B.Cu") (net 10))
 (segment (start 167.594157 114.75452) (end 150.67202 114.75452) (width 0.25) (layer "B.Cu") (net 10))
 (segment (start 150.67202 114.75452) (end 149.86 113.9425) (width 0.25) (layer "B.Cu") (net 10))
 (segment (start 168.195 107.95) (end 170.26 107.95) (width 0.25) (layer "B.Cu") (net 10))
 (segment (start 168.91 113.438677) (end 167.594157 114.75452) (width 0.25) (layer "B.Cu") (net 10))
 (segment (start 168.0425 109.855) (end 168.0425 108.1025) (width 0.25) (layer "B.Cu") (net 10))
 (segment (start 160.930498 108.359376) (end 160.930498 110.49) (width 0.25) (layer "F.Cu") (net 7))
 (segment (start 175.1 110.49) (end 159.222507 110.49) (width 0.25) (layer "F.Cu") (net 7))
 (segment (start 176.37 111.76) (end 175.1 110.49) (width 0.25) (layer "F.Cu") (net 7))
 (segment (start 158.507507 109.775) (end 153.115 109.775) (width 0.25) (layer "F.Cu") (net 7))
 (segment (start 180.34 110.49) (end 179.07 111.76) (width 0.25) (layer "F.Cu") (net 7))
 (segment (start 179.07 111.76) (end 176.37 111.76) (width 0.25) (layer "F.Cu") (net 7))
 (segment (start 153.115 109.775) (end 153.035 109.855) (width 0.25) (layer "F.Cu") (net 7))
 (segment (start 159.222507 110.49) (end 158.507507 109.775) (width 0.25) (layer "F.Cu") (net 7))
 (via (at 160.930498 108.359376) (size 0.8) (drill 0.4) (layers "F.Cu" "B.Cu") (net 7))
 (via (at 153.035 109.855) (size 0.8) (drill 0.4) (layers "F.Cu" "B.Cu") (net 7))
 (segment (start 159.239376 108.359376) (end 158.195 107.315) (width 0.25) (layer "B.Cu") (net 7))
 (segment (start 153.035 109.855) (end 151.765 109.855) (width 0.25) (layer "B.Cu") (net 7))
 (segment (start 175.895 109.855) (end 175.895 111.335614) (width 0.25) (layer "B.Cu") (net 7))
 (segment (start 175.895 111.335614) (end 176.319397 111.760011) (width 0.25) (layer "B.Cu") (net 7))
 (segment (start 179.069989 111.760011) (end 180.34 110.49) (width 0.25) (layer "B.Cu") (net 7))
 (segment (start 160.930498 108.359376) (end 159.239376 108.359376) (width 0.25) (layer "B.Cu") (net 7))
 (segment (start 176.319397 111.760011) (end 179.069989 111.760011) (width 0.25) (layer "B.Cu") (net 7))
 (segment (start 153.035 111.76) (end 152.6775 112.1175) (width 0.2) (layer "B.Cu") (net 11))
 (segment (start 160.995717 113.03) (end 160.396197 113.62952) (width 0.2) (layer "B.Cu") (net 11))
 (segment (start 161.6475 113.03) (end 160.995717 113.03) (width 0.2) (layer "B.Cu") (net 11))
 (segment (start 155.575 111.76) (end 154.435 111.76) (width 0.2) (layer "B.Cu") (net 11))
 (segment (start 154.435 111.76) (end 153.035 111.76) (width 0.2) (layer "B.Cu") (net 11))
 (segment (start 160.396197 113.62952) (end 157.44452 113.62952) (width 0.2) (layer "B.Cu") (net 11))
 (segment (start 152.6775 112.1175) (end 151.765 112.1175) (width 0.2) (layer "B.Cu") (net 11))
 (segment (start 157.44452 113.62952) (end 155.575 111.76) (width 0.2) (layer "B.Cu") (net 11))
 (segment (start 151.765 107.315) (end 152.56452 106.51548) (width 0.25) (layer "B.Cu") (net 8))
 (segment (start 152.56452 106.51548) (end 174.46048 106.51548) (width 0.25) (layer "B.Cu") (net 8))
 (segment (start 174.46048 106.51548) (end 175.895 107.95) (width 0.25) (layer "B.Cu") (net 8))
 (segment (start 175.895 107.95) (end 180.34 107.95) (width 0.25) (layer "B.Cu") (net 8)))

